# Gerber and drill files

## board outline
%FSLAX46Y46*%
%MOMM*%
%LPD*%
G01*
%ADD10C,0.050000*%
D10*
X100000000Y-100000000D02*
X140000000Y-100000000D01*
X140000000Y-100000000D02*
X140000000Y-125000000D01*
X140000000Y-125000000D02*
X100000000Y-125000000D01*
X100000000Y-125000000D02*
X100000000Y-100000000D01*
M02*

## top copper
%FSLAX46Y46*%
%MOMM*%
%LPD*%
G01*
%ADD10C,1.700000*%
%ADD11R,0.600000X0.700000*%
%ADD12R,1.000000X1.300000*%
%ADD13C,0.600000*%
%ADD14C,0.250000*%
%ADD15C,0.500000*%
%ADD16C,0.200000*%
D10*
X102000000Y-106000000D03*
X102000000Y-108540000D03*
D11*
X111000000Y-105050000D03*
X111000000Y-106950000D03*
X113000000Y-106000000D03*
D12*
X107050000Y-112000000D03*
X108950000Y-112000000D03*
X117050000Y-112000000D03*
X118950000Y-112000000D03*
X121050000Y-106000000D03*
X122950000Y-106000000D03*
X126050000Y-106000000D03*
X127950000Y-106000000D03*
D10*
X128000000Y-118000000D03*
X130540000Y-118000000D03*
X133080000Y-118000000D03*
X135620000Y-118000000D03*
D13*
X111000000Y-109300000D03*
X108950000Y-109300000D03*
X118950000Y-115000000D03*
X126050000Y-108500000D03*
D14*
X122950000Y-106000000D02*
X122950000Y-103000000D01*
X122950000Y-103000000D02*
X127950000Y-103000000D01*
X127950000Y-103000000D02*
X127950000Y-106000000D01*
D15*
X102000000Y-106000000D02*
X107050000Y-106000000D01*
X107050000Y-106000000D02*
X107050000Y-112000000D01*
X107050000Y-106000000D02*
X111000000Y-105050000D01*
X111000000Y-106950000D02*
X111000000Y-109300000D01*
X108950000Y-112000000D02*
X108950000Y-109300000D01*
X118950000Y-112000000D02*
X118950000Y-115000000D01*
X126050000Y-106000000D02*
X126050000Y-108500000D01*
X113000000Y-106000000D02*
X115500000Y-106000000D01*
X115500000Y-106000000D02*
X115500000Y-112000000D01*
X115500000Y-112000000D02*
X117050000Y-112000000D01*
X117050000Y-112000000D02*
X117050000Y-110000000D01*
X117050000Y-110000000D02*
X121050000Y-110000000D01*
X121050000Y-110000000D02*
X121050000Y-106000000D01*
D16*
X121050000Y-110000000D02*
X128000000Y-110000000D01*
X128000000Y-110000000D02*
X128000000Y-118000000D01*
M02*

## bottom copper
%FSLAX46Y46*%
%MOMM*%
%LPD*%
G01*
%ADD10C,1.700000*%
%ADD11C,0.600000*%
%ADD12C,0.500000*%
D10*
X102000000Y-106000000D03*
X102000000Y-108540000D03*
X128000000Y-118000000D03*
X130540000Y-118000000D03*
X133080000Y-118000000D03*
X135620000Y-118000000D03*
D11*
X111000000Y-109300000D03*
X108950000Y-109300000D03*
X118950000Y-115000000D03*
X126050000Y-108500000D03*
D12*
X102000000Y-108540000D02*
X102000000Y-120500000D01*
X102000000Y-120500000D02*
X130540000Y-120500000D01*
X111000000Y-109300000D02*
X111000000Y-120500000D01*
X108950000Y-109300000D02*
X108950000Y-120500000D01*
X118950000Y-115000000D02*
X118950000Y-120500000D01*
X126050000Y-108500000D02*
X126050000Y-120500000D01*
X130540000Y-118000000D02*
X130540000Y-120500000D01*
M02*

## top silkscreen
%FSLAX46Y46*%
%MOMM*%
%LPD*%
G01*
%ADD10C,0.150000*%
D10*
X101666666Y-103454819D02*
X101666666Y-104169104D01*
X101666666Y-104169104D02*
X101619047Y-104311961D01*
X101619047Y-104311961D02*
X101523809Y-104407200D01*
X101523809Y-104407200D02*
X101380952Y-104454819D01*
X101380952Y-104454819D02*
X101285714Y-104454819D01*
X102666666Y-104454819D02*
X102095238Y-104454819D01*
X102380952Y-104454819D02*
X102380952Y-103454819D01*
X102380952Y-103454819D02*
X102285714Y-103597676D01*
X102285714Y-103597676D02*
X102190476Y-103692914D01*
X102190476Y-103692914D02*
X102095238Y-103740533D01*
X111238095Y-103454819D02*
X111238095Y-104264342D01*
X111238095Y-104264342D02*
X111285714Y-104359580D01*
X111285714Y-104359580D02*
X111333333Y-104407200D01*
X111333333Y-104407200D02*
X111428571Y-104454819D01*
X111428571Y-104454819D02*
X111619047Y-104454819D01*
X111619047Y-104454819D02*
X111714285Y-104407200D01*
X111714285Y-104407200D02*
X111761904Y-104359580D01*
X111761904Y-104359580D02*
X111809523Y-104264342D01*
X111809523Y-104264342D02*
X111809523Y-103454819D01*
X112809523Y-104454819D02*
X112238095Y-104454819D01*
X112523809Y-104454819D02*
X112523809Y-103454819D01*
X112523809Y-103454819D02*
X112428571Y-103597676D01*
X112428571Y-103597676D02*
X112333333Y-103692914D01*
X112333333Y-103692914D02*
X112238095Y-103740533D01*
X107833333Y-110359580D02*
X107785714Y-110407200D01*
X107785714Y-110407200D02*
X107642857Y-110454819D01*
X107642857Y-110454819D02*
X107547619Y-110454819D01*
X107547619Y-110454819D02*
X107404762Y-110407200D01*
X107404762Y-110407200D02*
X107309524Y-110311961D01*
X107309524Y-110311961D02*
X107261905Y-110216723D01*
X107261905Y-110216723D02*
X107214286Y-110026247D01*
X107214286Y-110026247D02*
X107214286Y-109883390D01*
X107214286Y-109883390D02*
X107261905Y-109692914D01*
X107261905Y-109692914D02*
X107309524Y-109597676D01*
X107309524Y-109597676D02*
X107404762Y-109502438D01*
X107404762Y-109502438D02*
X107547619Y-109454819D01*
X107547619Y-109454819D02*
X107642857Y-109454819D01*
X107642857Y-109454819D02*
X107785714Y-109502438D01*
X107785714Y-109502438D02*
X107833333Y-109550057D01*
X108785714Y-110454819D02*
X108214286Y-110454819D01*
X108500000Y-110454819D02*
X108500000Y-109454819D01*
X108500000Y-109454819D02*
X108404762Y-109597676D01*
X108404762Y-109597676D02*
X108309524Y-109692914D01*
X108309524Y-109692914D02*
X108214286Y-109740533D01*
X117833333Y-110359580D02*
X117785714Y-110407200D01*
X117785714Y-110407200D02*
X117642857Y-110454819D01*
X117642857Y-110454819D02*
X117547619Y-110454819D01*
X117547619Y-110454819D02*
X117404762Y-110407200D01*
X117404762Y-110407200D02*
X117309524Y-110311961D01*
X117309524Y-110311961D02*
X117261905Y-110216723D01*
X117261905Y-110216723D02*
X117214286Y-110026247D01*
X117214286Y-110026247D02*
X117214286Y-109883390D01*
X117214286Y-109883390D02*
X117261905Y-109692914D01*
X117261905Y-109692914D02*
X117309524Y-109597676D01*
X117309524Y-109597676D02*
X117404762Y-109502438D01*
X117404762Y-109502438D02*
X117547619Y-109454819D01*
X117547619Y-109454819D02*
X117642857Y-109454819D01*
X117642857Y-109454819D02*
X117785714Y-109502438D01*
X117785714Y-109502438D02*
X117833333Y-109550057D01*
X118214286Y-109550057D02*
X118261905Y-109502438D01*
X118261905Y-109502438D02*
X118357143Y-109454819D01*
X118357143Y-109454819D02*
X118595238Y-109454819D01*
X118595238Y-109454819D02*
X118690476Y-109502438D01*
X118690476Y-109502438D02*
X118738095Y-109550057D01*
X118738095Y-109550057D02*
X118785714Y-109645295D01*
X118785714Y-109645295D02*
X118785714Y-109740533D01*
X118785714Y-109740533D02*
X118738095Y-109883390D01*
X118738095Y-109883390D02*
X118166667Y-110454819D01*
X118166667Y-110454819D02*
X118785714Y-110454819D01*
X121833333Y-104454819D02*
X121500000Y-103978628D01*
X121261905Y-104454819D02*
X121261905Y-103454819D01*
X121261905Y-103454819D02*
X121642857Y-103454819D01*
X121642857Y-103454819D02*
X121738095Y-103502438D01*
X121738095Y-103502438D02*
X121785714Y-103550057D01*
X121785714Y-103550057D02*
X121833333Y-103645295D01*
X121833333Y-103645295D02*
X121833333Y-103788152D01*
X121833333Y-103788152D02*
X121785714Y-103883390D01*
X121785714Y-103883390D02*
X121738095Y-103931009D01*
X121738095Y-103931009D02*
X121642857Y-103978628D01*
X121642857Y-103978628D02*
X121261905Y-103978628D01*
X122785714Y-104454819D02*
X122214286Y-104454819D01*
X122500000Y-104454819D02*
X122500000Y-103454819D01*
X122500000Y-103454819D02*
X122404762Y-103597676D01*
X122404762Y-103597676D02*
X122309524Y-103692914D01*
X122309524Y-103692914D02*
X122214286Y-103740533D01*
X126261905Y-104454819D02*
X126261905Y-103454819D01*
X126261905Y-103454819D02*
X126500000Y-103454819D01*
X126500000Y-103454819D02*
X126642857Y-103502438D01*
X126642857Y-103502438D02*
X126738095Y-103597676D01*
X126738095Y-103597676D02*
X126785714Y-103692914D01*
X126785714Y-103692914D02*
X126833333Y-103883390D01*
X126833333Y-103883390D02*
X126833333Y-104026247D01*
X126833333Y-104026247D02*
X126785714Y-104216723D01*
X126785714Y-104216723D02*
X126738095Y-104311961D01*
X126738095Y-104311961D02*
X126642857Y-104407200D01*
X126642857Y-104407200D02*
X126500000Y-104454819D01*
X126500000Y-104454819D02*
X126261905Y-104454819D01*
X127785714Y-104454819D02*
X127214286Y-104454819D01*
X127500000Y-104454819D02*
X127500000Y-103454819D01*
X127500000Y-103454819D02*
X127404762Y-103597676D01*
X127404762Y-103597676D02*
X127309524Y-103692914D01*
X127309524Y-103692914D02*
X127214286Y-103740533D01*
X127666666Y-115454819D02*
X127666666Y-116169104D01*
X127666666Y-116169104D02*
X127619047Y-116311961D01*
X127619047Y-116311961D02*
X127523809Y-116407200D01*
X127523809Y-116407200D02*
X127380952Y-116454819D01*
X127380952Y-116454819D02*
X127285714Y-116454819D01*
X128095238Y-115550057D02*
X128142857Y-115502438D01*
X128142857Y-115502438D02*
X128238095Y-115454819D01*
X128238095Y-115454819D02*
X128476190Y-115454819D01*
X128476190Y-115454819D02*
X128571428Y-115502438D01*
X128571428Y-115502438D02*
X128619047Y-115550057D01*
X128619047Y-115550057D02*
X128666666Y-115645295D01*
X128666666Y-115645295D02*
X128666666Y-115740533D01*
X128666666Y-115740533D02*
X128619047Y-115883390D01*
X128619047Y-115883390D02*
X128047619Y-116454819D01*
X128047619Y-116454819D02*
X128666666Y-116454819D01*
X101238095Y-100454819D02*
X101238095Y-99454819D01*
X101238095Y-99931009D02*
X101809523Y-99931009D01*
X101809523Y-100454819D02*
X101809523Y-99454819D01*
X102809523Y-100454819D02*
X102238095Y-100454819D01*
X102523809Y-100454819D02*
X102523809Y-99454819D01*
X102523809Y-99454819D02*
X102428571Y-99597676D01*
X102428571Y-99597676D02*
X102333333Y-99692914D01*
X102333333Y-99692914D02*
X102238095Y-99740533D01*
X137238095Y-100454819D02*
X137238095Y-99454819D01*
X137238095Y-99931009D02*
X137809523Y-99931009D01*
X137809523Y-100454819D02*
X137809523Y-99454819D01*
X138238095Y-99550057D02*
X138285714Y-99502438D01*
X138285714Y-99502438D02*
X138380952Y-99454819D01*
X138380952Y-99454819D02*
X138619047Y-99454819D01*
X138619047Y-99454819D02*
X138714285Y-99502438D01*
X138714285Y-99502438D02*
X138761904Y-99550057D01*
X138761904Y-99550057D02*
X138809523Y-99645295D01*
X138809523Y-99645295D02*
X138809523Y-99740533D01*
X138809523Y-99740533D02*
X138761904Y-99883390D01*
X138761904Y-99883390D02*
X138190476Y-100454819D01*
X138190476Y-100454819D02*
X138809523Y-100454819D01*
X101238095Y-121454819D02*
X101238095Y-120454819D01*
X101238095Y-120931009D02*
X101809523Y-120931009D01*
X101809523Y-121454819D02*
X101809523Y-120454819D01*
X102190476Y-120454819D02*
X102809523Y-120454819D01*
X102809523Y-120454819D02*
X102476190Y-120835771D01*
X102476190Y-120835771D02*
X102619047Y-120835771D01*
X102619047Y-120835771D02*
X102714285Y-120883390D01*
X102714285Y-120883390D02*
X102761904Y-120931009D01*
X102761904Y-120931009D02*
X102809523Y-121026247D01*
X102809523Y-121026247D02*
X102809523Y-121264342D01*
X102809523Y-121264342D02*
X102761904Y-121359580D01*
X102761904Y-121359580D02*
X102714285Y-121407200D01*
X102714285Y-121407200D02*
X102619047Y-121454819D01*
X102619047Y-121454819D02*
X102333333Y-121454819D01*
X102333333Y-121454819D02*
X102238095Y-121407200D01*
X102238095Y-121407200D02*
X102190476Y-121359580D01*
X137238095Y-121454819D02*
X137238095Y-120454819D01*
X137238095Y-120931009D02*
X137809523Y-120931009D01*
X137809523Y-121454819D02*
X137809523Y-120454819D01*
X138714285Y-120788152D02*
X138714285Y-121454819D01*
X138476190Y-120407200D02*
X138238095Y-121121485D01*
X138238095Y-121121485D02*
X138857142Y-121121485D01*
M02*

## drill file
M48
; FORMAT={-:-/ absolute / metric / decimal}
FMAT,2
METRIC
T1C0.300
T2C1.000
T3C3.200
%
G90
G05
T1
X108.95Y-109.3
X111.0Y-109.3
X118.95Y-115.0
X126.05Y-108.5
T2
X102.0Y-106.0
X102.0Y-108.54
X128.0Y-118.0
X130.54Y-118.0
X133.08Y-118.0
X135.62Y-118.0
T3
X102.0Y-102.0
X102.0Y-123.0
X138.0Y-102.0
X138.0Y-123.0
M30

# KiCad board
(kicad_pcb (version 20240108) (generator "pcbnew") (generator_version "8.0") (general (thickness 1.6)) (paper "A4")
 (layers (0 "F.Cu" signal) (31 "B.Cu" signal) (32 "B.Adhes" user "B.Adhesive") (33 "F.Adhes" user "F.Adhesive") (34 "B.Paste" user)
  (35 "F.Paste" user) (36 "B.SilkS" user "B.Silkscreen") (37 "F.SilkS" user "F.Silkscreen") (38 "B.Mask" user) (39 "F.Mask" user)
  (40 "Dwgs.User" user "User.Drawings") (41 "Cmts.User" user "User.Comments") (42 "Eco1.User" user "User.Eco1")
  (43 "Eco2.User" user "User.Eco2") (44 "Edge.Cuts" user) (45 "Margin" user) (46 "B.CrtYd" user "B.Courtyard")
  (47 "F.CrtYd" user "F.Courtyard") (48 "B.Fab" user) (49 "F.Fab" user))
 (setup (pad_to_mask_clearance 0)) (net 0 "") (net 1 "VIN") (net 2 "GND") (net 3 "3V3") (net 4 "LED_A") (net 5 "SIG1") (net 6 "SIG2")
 (gr_line (start 100 100) (end 140 100) (stroke (width 0.05) (type default)) (layer "Edge.Cuts"))
 (gr_line (start 140 100) (end 140 125) (stroke (width 0.05) (type default)) (layer "Edge.Cuts"))
 (gr_line (start 140 125) (end 100 125) (stroke (width 0.05) (type default)) (layer "Edge.Cuts"))
 (gr_line (start 100 125) (end 100 100) (stroke (width 0.05) (type default)) (layer "Edge.Cuts"))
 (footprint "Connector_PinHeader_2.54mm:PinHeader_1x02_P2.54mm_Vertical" (layer "F.Cu") (at 102 106)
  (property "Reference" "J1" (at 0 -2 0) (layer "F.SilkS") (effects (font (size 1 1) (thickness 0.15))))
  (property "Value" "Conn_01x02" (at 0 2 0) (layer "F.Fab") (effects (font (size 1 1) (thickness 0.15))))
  (pad "1" thru_hole circle (at 0 0) (size 1.7 1.7) (drill 1) (layers "*.Cu" "*.Mask") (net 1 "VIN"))
  (pad "2" thru_hole circle (at 0 2.54) (size 1.7 1.7) (drill 1) (layers "*.Cu" "*.Mask") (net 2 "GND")))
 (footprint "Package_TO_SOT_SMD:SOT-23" (layer "F.Cu") (at 112 106)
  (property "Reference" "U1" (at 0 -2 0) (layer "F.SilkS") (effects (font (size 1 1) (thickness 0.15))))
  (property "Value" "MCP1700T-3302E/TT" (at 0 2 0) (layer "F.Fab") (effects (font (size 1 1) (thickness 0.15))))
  (pad "1" smd rect (at -1 -0.95) (size 0.6 0.7) (layers "F.Cu" "F.Paste" "F.Mask") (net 1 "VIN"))
  (pad "2" smd rect (at -1 0.95) (size 0.6 0.7) (layers "F.Cu" "F.Paste" "F.Mask") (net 2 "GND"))
  (pad "3" smd rect (at 1 0) (size 0.6 0.7) (layers "F.Cu" "F.Paste" "F.Mask") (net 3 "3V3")))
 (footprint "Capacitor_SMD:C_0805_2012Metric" (layer "F.Cu") (at 108 112)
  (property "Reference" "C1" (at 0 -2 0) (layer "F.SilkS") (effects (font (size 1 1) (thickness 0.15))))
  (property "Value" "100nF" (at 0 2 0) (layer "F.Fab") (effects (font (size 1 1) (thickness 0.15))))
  (pad "1" smd rect (at -0.95 0) (size 1 1.3) (layers "F.Cu" "F.Paste" "F.Mask") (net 1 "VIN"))
  (pad "2" smd rect (at 0.95 0) (size 1 1.3) (layers "F.Cu" "F.Paste" "F.Mask") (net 2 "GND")))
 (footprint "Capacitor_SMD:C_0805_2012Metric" (layer "F.Cu") (at 118 112)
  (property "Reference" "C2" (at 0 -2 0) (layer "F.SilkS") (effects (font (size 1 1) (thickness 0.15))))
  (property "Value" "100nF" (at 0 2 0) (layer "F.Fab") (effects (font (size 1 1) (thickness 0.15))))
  (pad "1" smd rect (at -0.95 0) (size 1 1.3) (layers "F.Cu" "F.Paste" "F.Mask") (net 3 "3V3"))
  (pad "2" smd rect (at 0.95 0) (size 1 1.3) (layers "F.Cu" "F.Paste" "F.Mask") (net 2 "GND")))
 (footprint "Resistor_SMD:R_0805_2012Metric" (layer "F.Cu") (at 122 106)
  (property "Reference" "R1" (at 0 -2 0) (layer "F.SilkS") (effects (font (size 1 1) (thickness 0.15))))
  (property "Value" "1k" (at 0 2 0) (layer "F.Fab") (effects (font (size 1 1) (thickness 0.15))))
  (pad "1" smd rect (at -0.95 0) (size 1 1.3) (layers "F.Cu" "F.Paste" "F.Mask") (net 3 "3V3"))
  (pad "2" smd rect (at 0.95 0) (size 1 1.3) (layers "F.Cu" "F.Paste" "F.Mask") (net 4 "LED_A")))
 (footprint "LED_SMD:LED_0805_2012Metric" (layer "F.Cu") (at 127 106)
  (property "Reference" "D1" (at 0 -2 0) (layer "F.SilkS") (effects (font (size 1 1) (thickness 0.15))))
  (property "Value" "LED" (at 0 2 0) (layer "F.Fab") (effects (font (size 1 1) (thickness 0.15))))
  (pad "1" smd rect (at -0.95 0) (size 1 1.3) (layers "F.Cu" "F.Paste" "F.Mask") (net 2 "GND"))
  (pad "2" smd rect (at 0.95 0) (size 1 1.3) (layers "F.Cu" "F.Paste" "F.Mask") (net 4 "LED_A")))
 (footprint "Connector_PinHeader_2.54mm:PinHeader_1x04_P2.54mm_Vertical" (layer "F.Cu") (at 128 118)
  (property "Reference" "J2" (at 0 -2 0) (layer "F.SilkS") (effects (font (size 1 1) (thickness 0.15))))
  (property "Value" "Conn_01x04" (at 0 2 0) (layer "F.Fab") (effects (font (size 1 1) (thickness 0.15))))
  (pad "1" thru_hole circle (at 0 0) (size 1.7 1.7) (drill 1) (layers "*.Cu" "*.Mask") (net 3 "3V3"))
  (pad "2" thru_hole circle (at 2.54 0) (size 1.7 1.7) (drill 1) (layers "*.Cu" "*.Mask") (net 2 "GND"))
  (pad "3" thru_hole circle (at 5.08 0) (size 1.7 1.7) (drill 1) (layers "*.Cu" "*.Mask") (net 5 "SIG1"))
  (pad "4" thru_hole circle (at 7.62 0) (size 1.7 1.7) (drill 1) (layers "*.Cu" "*.Mask") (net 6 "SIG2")))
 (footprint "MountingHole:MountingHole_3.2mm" (layer "F.Cu") (at 102 102)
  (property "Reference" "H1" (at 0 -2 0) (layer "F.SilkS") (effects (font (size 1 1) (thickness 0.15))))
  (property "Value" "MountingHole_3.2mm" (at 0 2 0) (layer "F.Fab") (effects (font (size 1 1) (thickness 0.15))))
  (pad "1" np_thru_hole circle (at 0 0) (size 3.2 3.2) (drill 3.2) (layers "*.Cu" "*.Mask")))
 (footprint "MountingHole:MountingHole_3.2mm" (layer "F.Cu") (at 138 102)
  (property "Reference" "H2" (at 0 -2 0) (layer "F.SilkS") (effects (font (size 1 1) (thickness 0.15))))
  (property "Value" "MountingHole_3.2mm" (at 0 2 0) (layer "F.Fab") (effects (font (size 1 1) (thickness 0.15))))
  (pad "1" np_thru_hole circle (at 0 0) (size 3.2 3.2) (drill 3.2) (layers "*.Cu" "*.Mask")))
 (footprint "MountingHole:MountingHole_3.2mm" (layer "F.Cu") (at 102 123)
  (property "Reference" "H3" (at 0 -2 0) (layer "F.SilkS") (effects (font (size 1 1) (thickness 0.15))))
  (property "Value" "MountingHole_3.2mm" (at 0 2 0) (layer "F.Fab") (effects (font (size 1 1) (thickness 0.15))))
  (pad "1" np_thru_hole circle (at 0 0) (size 3.2 3.2) (drill 3.2) (layers "*.Cu" "*.Mask")))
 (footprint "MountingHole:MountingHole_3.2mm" (layer "F.Cu") (at 138 123)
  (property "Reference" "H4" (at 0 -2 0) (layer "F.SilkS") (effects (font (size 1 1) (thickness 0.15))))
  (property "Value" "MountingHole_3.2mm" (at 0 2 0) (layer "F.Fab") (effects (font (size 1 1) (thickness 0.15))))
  (pad "1" np_thru_hole circle (at 0 0) (size 3.2 3.2) (drill 3.2) (layers "*.Cu" "*.Mask")))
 (segment (start 122.95 106) (end 122.95 103) (width 0.25) (layer "F.Cu") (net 4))
 (segment (start 122.95 103) (end 127.95 103) (width 0.25) (layer "F.Cu") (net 4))
 (segment (start 127.95 103) (end 127.95 106) (width 0.25) (layer "F.Cu") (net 4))
 (segment (start 102 106) (end 107.05 106) (width 0.5) (layer "F.Cu") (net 1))
 (segment (start 107.05 106) (end 107.05 112) (width 0.5) (layer "F.Cu") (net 1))
 (segment (start 107.05 106) (end 111 105.05) (width 0.5) (layer "F.Cu") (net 1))
 (segment (start 111 106.95) (end 111 109.3) (width 0.5) (layer "F.Cu") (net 2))
 (segment (start 108.95 112) (end 108.95 109.3) (width 0.5) (layer "F.Cu") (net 2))
 (segment (start 118.95 112) (end 118.95 115) (width 0.5) (layer "F.Cu") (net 2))
 (segment (start 126.05 106) (end 126.05 108.5) (width 0.5) (layer "F.Cu") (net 2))
 (segment (start 113 106) (end 115.5 106) (width 0.5) (layer "F.Cu") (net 3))
 (segment (start 115.5 106) (end 115.5 112) (width 0.5) (layer "F.Cu") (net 3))
 (segment (start 115.5 112) (end 117.05 112) (width 0.5) (layer "F.Cu") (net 3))
 (segment (start 117.05 112) (end 117.05 110) (width 0.5) (layer "F.Cu") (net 3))
 (segment (start 117.05 110) (end 121.05 110) (width 0.5) (layer "F.Cu") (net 3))
 (segment (start 121.05 110) (end 121.05 106) (width 0.5) (layer "F.Cu") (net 3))
 (segment (start 121.05 110) (end 128 110) (width 0.2) (layer "F.Cu") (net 3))
 (segment (start 128 110) (end 128 118) (width 0.2) (layer "F.Cu") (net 3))
 (segment (start 102 108.54) (end 102 120.5) (width 0.5) (layer "B.Cu") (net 2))
 (segment (start 102 120.5) (end 130.54 120.5) (width 0.5) (layer "B.Cu") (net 2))
 (segment (start 111 109.3) (end 111 120.5) (width 0.5) (layer "B.Cu") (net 2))
 (segment (start 108.95 109.3) (end 108.95 120.5) (width 0.5) (layer "B.Cu") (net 2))
 (segment (start 118.95 115) (end 118.95 120.5) (width 0.5) (layer "B.Cu") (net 2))
 (segment (start 126.05 108.5) (end 126.05 120.5) (width 0.5) (layer "B.Cu") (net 2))
 (segment (start 130.54 118) (end 130.54 120.5) (width 0.5) (layer "B.Cu") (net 2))
 (via (at 111 109.3) (size 0.6) (drill 0.3) (layers "F.Cu" "B.Cu") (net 2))
 (via (at 108.95 109.3) (size 0.6) (drill 0.3) (layers "F.Cu" "B.Cu") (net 2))
 (via (at 118.95 115) (size 0.6) (drill 0.3) (layers "F.Cu" "B.Cu") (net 2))
 (via (at 126.05 108.5) (size 0.6) (drill 0.3) (layers "F.Cu" "B.Cu") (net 2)))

